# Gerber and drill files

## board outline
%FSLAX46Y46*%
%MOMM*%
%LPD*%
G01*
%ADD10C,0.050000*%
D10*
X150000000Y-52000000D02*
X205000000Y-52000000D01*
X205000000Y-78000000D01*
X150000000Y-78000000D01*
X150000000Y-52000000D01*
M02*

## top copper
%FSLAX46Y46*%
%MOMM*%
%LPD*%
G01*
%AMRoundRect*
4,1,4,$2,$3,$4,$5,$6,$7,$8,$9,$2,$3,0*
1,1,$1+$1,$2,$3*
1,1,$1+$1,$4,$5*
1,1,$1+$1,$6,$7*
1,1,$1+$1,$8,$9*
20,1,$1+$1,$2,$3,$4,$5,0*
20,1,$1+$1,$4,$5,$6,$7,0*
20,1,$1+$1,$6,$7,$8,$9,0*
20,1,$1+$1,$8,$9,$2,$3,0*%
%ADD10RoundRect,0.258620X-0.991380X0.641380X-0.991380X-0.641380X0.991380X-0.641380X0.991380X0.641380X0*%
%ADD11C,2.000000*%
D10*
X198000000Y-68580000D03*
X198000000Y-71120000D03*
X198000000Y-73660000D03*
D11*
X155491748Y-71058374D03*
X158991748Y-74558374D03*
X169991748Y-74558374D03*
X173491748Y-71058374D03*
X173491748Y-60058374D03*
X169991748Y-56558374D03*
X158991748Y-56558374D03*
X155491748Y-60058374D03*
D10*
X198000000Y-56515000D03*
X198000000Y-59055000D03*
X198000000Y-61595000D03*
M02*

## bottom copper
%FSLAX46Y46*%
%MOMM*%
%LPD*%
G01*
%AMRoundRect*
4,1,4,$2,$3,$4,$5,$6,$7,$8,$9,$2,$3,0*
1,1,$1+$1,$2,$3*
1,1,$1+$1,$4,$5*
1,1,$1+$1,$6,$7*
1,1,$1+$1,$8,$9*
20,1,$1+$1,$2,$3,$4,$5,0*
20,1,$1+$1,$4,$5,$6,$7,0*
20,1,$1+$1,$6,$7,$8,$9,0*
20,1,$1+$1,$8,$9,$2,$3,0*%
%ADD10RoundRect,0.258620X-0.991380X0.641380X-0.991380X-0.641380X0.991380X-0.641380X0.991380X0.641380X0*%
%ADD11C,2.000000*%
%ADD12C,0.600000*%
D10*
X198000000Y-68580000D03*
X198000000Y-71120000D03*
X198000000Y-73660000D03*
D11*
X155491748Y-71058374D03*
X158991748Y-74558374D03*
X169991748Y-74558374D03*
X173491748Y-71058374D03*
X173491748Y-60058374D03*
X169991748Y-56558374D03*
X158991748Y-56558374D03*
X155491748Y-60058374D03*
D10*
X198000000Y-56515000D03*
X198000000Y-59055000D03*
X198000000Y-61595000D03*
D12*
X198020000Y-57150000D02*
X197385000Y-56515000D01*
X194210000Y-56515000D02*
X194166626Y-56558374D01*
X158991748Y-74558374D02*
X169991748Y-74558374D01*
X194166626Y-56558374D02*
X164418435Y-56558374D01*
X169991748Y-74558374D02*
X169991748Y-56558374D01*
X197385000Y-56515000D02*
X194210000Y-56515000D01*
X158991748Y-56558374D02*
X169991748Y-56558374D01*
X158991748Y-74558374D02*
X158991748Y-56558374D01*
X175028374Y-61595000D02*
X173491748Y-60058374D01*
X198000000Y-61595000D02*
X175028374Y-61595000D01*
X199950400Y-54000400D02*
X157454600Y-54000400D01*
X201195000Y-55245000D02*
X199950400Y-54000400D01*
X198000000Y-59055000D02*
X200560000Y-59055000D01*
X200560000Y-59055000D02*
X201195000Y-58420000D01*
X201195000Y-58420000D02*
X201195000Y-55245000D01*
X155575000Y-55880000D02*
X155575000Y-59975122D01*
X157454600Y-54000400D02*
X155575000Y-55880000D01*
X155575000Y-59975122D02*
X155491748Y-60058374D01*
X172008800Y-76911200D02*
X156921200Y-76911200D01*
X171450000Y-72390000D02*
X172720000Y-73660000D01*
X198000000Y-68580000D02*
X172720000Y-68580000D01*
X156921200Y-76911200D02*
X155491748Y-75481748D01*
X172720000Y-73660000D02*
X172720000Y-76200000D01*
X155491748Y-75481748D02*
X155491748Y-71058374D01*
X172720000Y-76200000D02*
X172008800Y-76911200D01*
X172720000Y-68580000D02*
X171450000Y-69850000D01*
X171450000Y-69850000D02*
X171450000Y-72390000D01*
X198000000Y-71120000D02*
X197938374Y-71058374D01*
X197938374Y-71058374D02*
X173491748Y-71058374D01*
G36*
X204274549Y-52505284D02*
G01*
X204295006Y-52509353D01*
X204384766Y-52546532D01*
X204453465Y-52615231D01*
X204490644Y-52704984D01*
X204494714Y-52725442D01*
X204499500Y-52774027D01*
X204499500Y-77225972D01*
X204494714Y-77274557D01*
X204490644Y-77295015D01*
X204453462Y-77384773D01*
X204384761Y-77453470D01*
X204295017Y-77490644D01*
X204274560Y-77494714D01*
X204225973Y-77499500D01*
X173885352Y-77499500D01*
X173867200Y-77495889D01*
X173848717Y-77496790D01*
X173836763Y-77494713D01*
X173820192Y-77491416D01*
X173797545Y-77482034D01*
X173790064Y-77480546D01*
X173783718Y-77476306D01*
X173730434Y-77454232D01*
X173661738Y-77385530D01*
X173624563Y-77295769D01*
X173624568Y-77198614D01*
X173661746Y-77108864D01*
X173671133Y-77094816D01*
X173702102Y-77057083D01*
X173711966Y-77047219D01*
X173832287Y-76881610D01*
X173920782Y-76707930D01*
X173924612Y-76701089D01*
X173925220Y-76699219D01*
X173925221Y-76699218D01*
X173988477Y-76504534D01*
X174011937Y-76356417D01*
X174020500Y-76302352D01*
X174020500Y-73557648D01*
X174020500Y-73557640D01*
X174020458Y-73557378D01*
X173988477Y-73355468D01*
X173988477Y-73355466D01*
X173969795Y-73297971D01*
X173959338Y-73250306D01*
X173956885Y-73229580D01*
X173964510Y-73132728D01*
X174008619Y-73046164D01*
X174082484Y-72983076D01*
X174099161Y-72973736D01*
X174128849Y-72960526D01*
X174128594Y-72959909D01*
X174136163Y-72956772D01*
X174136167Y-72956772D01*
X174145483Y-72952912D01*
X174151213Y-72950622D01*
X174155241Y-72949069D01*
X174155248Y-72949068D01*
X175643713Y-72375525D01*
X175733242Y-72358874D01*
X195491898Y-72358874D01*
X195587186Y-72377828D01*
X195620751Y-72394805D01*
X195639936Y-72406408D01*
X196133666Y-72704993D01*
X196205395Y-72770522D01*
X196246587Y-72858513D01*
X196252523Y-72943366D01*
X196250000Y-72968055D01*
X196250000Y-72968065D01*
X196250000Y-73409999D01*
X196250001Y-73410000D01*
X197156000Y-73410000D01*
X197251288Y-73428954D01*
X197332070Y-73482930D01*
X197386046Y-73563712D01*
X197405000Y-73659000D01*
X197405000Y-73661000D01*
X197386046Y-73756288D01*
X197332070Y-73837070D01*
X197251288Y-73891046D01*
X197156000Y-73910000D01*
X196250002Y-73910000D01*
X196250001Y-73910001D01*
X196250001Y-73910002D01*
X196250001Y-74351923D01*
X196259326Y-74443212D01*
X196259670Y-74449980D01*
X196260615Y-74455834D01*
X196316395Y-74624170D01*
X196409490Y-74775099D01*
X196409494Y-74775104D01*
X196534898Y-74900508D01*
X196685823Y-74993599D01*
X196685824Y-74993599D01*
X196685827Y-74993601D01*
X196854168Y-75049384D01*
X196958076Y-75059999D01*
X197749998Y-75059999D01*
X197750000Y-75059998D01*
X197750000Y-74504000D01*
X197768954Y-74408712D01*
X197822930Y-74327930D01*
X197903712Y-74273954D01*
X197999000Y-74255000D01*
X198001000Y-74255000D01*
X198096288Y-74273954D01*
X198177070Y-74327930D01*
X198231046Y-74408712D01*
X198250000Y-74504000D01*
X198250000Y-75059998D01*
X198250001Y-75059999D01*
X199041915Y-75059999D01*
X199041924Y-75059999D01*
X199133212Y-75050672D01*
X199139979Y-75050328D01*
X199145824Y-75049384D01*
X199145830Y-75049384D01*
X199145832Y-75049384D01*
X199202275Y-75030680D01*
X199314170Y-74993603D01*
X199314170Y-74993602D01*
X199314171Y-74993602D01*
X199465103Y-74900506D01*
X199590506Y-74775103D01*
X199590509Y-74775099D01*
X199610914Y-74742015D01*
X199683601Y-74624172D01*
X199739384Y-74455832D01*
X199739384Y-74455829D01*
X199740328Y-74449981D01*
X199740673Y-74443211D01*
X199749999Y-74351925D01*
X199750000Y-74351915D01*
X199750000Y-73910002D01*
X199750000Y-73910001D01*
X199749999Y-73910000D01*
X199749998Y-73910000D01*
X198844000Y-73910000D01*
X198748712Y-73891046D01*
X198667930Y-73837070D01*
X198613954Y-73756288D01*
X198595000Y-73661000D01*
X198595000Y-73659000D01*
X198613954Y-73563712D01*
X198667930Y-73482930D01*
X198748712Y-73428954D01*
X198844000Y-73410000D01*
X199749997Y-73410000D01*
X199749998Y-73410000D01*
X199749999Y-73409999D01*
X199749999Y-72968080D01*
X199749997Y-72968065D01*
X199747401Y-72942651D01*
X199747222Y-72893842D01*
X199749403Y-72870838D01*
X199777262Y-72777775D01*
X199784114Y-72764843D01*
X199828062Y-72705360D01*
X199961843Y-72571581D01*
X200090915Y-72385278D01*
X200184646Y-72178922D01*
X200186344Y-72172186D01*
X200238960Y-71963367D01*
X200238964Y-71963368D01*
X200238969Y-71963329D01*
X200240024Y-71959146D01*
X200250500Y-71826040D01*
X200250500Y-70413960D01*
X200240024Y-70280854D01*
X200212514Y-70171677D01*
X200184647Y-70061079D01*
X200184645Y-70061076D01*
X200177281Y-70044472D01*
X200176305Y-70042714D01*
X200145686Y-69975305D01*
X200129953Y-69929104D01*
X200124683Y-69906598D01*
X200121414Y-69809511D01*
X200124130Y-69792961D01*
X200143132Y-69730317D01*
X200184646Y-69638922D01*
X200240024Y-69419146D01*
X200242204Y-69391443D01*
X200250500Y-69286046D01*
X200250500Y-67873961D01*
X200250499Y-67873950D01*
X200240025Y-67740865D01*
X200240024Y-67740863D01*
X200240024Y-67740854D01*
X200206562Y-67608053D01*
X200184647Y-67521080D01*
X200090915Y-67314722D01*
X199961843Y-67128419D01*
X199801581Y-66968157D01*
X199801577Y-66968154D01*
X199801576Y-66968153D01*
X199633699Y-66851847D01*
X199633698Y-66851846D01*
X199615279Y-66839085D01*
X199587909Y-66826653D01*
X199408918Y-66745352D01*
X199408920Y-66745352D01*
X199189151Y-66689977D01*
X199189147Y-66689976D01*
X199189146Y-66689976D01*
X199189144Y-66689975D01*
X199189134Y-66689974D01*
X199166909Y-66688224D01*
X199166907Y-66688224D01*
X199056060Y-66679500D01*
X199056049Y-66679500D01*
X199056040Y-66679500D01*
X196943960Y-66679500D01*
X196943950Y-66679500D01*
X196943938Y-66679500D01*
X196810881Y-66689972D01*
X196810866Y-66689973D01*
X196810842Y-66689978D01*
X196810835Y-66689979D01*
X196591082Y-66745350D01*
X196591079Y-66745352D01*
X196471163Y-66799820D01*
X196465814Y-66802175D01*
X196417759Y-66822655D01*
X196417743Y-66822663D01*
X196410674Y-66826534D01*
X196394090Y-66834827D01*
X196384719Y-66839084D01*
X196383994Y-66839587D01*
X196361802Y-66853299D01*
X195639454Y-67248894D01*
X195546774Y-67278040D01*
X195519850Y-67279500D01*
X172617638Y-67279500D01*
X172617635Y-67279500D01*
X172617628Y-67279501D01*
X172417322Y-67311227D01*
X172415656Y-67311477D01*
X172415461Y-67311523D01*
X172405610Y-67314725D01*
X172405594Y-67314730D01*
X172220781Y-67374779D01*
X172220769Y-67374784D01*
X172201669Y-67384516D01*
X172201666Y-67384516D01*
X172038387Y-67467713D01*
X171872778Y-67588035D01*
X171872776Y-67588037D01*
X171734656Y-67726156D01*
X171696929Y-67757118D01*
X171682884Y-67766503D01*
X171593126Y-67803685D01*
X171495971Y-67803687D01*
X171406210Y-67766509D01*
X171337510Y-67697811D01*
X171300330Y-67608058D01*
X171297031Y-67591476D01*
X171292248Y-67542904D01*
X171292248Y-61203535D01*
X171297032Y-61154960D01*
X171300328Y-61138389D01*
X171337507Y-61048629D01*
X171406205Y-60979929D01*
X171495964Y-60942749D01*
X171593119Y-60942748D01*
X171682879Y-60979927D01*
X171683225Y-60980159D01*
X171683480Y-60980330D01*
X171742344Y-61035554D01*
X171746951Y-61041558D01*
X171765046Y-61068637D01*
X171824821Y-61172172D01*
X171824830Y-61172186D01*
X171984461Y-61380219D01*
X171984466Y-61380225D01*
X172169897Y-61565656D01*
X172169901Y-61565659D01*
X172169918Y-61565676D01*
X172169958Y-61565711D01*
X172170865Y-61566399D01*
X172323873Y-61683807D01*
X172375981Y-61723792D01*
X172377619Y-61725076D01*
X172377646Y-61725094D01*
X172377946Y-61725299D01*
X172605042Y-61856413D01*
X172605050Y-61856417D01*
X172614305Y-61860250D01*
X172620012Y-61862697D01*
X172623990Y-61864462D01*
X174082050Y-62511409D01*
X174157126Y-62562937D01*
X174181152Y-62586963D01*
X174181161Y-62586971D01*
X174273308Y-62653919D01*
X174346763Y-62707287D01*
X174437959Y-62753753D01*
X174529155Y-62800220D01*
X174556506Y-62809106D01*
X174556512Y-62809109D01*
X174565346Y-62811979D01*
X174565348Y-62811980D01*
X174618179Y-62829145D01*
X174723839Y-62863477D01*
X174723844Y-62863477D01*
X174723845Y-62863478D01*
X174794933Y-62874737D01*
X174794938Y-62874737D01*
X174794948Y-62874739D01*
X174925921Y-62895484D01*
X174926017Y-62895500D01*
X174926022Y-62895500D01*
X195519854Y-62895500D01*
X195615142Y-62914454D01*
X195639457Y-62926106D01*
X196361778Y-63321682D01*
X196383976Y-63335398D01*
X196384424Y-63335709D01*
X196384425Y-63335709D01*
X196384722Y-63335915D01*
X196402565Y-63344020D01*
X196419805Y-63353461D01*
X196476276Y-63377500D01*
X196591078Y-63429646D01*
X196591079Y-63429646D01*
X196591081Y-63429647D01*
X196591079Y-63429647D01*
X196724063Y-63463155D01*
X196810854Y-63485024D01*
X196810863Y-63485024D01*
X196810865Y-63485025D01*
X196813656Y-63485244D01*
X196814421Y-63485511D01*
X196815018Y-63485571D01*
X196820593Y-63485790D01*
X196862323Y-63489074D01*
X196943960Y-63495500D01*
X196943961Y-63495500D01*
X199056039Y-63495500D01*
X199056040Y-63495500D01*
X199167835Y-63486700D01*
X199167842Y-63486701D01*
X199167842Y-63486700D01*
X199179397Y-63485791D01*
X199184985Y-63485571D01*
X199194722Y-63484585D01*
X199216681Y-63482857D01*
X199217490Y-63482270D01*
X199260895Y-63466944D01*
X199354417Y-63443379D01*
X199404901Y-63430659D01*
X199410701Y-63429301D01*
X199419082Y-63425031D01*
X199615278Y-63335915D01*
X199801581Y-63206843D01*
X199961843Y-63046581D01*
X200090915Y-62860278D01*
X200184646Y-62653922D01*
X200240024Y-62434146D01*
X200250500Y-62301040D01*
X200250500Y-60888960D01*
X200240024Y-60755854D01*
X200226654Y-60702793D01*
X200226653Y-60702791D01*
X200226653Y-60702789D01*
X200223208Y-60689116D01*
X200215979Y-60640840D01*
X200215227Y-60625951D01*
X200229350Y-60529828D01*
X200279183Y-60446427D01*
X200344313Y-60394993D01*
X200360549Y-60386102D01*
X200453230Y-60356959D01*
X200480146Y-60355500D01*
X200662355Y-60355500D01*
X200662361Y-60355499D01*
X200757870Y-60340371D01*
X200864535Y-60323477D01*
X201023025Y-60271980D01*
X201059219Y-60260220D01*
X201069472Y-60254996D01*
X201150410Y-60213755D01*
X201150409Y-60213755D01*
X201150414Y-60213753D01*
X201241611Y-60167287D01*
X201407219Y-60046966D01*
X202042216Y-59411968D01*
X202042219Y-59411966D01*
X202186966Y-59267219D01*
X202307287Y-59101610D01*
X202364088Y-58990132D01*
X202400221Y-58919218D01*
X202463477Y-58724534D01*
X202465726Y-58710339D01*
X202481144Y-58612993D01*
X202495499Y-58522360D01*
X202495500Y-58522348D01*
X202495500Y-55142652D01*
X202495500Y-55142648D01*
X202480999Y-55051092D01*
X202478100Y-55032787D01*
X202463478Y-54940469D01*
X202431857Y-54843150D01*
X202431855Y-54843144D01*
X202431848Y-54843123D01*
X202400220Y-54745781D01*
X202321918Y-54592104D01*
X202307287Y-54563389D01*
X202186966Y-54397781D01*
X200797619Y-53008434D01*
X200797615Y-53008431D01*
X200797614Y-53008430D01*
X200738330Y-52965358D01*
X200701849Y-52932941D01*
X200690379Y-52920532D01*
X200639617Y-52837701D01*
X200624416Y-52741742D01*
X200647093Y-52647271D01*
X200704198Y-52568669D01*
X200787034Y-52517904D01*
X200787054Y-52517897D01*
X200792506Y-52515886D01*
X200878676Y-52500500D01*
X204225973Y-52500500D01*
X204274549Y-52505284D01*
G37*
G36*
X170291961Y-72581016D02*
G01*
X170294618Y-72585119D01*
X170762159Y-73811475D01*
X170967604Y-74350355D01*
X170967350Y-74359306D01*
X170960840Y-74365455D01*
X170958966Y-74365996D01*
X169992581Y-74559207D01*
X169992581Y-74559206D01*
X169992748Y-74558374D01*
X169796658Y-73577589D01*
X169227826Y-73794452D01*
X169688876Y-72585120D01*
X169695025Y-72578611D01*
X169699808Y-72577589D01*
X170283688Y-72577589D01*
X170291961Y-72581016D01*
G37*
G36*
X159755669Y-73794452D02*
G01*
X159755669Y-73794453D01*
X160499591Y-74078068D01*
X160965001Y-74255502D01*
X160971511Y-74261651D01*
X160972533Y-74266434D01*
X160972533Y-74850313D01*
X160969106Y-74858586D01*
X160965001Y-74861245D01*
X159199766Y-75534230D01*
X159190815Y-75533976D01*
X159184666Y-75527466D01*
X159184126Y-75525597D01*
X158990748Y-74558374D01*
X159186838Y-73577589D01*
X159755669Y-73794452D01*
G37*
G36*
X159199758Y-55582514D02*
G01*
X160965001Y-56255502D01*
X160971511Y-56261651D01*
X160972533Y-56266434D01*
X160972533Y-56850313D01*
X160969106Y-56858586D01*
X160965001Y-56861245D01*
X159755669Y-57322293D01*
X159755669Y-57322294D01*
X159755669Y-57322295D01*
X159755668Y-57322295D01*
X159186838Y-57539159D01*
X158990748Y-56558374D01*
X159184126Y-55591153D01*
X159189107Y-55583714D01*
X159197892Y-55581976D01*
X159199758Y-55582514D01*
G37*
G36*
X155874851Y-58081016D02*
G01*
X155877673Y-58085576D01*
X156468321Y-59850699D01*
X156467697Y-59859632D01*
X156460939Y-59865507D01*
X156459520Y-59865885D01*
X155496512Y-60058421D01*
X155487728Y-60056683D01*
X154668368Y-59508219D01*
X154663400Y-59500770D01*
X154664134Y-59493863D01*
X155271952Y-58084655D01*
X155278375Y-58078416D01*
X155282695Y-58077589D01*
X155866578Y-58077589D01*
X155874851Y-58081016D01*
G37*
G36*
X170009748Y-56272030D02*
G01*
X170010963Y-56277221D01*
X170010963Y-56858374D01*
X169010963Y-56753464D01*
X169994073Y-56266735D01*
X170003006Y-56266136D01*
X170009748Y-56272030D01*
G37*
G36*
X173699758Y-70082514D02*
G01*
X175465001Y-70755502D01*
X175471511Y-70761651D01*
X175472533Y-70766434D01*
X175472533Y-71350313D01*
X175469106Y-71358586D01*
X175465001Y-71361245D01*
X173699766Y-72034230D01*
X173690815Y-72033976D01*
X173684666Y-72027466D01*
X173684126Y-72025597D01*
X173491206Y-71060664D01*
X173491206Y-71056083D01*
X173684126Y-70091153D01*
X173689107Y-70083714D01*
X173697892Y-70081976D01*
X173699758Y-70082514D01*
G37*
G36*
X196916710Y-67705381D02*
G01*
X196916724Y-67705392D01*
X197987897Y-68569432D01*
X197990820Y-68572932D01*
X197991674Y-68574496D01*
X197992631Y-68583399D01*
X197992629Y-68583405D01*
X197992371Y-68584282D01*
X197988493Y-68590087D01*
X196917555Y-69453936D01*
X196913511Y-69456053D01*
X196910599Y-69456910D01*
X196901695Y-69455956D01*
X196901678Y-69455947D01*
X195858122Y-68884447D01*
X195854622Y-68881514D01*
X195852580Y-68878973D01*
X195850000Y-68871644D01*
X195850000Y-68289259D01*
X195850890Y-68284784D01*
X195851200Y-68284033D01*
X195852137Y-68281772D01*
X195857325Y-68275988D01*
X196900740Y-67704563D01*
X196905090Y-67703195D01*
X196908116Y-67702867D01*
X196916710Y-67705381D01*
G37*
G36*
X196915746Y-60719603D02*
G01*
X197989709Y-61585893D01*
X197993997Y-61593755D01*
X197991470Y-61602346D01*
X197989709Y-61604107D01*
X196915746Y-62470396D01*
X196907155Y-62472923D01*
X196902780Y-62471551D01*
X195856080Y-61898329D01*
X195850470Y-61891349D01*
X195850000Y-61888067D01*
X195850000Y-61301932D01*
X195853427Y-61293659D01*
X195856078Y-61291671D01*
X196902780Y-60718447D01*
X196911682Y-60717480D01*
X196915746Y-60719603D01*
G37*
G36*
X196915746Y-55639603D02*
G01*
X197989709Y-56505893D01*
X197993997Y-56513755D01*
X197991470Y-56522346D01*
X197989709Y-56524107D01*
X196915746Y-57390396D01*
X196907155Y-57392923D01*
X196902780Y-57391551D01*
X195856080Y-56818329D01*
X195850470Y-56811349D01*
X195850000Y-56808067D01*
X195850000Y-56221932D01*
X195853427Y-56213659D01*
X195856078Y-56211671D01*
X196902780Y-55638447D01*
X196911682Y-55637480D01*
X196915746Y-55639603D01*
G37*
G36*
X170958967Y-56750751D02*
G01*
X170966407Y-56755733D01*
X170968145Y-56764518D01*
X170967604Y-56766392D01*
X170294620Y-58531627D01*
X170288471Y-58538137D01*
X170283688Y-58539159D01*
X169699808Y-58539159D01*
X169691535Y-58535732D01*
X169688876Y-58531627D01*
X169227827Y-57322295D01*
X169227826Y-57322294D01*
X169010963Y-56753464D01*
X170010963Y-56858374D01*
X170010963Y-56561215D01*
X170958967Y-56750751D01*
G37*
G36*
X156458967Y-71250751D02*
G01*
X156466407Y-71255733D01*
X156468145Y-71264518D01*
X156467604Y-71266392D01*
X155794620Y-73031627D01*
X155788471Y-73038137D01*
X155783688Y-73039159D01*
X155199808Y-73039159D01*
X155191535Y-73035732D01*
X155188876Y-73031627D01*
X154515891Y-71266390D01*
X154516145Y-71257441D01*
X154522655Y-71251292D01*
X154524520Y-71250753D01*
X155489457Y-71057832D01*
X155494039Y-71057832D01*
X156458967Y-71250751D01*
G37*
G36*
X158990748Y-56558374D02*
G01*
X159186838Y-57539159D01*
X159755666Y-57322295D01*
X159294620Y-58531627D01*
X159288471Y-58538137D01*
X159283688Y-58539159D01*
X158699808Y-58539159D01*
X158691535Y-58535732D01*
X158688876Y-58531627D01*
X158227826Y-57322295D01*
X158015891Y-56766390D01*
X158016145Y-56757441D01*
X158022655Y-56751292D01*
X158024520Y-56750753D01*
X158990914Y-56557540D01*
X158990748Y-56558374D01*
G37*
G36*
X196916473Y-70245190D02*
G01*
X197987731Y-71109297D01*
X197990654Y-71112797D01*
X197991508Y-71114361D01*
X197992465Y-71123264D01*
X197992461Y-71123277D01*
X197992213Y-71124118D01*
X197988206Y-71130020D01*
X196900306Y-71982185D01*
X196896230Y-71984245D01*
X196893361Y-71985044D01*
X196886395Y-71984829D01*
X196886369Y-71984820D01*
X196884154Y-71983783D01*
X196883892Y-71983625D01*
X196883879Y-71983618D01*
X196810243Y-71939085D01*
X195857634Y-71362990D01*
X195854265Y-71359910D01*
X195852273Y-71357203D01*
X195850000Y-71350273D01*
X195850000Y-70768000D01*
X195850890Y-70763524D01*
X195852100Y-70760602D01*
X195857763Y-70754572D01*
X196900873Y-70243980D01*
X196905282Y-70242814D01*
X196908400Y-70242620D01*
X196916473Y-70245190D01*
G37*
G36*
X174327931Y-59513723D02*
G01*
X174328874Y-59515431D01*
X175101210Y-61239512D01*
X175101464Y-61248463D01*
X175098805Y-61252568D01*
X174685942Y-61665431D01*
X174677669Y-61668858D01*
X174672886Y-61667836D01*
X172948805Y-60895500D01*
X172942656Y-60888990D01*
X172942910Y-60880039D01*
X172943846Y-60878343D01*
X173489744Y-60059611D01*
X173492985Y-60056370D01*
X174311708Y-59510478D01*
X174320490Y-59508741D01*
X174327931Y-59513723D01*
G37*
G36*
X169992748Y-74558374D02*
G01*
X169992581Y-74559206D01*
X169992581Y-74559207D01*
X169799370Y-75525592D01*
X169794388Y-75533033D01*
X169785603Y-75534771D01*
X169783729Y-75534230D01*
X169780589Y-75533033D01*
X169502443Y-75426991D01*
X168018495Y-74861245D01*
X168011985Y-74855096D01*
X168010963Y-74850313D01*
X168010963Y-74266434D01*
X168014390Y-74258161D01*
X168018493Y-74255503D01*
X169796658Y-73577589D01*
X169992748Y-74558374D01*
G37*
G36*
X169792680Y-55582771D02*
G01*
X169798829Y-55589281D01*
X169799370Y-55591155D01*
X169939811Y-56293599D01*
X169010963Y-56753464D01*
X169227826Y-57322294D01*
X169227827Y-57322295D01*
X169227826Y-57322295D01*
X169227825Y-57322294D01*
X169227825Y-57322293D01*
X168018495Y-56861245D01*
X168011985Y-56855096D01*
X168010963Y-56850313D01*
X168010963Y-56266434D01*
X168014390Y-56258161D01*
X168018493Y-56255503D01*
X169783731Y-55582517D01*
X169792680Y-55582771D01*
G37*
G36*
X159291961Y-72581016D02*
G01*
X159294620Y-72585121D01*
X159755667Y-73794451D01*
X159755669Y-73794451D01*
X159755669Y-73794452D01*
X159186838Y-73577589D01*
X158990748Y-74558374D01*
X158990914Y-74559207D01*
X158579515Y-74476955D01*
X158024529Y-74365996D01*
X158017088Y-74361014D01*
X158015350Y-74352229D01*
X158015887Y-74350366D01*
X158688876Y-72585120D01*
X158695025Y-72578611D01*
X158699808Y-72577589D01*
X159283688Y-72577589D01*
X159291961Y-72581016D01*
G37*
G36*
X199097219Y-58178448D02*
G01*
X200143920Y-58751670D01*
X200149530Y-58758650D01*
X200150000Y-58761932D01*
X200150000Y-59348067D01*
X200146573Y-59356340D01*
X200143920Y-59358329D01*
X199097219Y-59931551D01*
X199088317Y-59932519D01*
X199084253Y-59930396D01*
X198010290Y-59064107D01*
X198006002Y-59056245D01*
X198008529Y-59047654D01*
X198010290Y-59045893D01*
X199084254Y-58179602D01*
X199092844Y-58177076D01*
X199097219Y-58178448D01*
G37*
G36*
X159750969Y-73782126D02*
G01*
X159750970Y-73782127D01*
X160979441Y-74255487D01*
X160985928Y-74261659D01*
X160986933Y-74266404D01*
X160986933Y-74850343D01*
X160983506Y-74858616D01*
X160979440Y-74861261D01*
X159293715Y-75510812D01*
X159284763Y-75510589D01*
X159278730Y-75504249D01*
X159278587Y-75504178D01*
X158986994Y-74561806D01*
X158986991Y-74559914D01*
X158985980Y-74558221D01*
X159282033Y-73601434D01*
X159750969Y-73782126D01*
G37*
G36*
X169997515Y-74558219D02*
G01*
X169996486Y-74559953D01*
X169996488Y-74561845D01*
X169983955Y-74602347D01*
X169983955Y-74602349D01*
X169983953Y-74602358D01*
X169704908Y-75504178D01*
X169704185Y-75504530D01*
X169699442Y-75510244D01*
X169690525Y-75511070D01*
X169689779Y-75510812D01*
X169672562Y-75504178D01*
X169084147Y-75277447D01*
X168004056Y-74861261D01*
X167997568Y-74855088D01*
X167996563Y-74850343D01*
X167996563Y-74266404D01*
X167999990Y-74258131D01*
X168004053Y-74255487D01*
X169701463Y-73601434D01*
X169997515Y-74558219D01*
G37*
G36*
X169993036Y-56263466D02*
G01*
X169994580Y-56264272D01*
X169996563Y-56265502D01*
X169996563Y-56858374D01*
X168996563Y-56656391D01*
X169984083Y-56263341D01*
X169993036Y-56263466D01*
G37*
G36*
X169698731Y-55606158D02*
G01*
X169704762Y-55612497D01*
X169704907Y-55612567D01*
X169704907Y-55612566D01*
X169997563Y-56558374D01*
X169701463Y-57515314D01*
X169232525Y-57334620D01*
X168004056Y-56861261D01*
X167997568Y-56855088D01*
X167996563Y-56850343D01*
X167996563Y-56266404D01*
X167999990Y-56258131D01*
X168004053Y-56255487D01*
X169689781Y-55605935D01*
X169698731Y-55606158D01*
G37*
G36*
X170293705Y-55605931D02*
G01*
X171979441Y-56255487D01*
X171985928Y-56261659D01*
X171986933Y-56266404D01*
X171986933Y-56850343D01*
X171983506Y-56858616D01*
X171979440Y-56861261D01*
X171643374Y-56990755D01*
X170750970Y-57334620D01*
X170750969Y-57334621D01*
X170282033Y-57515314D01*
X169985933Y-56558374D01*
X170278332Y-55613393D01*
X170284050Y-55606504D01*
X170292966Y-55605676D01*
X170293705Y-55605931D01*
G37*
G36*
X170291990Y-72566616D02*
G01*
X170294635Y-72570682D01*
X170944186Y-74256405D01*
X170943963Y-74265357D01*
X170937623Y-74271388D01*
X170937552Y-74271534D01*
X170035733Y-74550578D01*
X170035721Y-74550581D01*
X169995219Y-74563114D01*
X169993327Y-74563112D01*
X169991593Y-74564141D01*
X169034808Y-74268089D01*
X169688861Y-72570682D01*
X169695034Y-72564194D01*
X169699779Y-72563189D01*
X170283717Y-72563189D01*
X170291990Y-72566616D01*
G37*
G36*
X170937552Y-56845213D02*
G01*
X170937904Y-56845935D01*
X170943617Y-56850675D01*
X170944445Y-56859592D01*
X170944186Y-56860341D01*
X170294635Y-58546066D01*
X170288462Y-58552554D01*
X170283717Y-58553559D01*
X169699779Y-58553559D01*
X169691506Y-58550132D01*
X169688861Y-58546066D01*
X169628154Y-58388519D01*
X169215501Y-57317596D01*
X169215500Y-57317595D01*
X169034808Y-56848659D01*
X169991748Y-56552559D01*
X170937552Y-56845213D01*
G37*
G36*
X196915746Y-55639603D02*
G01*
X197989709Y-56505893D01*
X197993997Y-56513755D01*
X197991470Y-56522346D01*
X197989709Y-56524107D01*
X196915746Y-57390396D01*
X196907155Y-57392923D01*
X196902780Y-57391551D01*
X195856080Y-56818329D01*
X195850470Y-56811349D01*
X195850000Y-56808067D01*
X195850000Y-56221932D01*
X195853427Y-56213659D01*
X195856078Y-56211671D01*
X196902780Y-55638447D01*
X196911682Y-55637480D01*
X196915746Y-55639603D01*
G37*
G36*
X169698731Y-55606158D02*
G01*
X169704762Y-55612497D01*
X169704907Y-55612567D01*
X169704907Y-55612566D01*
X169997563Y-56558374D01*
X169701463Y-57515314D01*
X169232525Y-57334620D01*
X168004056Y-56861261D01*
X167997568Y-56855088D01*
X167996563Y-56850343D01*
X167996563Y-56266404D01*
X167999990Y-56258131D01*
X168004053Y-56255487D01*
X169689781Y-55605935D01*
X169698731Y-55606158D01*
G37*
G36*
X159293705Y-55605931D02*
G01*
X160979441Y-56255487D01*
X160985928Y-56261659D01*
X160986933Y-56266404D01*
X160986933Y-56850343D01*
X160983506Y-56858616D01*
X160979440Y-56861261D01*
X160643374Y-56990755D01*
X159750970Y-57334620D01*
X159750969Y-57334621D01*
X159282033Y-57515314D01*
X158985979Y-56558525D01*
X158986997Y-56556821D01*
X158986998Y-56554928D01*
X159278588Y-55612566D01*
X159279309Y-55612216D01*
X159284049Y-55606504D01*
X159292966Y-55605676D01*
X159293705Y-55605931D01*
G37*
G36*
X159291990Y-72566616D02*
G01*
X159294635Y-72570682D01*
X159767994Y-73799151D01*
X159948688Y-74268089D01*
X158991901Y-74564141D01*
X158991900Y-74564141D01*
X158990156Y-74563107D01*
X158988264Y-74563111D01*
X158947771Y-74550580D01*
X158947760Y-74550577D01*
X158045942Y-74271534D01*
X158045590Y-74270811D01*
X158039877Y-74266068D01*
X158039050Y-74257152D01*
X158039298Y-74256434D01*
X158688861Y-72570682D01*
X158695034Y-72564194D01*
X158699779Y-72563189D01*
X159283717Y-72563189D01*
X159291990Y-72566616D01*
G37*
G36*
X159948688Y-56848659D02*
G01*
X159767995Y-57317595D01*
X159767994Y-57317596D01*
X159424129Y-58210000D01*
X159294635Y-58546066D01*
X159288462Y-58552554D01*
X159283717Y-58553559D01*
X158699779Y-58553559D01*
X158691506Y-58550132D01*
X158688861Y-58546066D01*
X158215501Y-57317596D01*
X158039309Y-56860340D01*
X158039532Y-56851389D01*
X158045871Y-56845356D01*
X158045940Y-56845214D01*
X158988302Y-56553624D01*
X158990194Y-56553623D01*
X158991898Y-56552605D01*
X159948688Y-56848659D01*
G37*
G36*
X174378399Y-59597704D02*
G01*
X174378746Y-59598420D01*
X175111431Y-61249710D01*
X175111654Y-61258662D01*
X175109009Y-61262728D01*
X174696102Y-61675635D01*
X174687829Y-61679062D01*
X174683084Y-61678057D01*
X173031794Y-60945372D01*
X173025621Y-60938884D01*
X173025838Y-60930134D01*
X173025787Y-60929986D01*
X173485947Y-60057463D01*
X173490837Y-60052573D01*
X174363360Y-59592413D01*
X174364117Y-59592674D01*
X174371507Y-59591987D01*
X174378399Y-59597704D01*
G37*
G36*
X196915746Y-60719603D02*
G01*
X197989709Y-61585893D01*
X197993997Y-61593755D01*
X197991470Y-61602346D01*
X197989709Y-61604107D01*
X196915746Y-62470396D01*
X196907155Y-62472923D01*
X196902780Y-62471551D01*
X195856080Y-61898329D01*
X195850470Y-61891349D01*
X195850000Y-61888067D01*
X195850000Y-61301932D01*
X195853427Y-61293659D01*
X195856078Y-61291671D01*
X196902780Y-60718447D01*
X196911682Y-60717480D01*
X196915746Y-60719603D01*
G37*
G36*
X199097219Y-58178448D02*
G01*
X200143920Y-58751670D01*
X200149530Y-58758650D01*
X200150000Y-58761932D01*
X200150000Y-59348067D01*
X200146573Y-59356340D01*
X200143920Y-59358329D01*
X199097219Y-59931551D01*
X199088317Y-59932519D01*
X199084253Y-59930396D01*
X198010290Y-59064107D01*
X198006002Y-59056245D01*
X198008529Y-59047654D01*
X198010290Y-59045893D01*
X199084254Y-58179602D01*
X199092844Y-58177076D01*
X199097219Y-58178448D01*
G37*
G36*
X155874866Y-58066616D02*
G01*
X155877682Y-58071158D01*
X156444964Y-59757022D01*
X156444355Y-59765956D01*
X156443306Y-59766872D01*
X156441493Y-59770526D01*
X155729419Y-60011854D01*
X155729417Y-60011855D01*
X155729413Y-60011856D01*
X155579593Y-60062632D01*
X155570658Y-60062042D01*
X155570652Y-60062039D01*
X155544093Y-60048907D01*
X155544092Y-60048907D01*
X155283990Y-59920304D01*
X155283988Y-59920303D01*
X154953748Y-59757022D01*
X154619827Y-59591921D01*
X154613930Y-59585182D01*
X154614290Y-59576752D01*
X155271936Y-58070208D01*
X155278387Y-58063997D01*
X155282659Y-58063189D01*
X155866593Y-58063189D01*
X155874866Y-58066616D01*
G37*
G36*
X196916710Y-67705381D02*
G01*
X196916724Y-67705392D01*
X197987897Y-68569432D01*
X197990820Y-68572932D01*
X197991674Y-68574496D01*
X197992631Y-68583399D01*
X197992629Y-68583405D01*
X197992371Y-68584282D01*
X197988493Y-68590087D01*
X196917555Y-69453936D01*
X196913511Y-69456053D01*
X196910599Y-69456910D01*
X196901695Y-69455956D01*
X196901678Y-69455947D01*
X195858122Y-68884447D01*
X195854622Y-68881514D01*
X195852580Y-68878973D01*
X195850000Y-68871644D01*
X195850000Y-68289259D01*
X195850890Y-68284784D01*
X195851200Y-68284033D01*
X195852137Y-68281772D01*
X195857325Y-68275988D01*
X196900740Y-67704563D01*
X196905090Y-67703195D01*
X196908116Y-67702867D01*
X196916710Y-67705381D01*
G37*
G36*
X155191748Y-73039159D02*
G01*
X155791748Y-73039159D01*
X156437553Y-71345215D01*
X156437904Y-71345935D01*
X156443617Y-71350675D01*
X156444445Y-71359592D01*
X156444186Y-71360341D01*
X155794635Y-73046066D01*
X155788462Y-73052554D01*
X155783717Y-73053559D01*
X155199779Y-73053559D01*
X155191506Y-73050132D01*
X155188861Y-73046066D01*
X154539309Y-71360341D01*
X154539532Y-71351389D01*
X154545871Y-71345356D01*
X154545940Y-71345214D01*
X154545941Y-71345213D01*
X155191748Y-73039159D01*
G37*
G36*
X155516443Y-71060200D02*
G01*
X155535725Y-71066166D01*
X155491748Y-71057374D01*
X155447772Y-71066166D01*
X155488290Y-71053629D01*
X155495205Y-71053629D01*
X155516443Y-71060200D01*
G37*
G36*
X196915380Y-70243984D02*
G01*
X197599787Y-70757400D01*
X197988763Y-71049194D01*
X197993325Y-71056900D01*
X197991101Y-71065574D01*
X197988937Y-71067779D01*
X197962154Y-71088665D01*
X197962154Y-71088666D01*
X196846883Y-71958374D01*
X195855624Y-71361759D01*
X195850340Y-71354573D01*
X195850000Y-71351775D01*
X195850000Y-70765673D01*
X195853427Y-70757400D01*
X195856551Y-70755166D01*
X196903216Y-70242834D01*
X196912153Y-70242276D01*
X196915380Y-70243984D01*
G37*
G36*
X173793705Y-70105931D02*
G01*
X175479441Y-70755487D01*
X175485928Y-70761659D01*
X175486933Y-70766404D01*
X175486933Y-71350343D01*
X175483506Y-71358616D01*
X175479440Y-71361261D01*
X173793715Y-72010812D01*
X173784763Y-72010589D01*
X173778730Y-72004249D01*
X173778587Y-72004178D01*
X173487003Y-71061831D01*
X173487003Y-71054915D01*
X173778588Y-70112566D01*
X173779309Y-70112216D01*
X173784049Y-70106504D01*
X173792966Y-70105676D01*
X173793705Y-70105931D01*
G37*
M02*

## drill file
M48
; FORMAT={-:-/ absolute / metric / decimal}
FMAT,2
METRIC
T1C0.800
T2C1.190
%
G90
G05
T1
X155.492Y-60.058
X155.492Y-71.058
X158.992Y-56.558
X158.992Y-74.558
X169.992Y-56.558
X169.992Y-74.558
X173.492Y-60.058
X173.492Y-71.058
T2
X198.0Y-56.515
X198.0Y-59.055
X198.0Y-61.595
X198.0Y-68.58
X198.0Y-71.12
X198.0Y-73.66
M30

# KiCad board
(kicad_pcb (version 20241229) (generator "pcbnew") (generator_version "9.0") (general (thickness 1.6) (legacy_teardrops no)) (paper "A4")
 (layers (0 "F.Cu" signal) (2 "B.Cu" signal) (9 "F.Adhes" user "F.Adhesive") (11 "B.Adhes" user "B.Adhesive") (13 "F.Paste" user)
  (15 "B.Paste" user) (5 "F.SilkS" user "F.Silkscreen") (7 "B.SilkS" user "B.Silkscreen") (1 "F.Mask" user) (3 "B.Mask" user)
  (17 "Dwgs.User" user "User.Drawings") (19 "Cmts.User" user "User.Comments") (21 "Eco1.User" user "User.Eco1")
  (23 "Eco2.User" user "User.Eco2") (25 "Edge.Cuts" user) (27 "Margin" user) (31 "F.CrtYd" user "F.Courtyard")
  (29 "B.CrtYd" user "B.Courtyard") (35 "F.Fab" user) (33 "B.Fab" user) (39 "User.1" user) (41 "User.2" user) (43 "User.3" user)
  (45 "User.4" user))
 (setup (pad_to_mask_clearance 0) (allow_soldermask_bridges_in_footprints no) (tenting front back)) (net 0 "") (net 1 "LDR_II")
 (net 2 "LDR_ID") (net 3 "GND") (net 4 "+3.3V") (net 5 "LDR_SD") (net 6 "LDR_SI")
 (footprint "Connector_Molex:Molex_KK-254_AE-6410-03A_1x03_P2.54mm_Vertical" (layer "F.Cu") (at 198 68.58 -90)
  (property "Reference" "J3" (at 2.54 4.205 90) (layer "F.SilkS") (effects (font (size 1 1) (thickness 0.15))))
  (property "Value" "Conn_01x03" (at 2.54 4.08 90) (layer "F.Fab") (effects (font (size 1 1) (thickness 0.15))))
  (pad "1" thru_hole roundrect (at 0 0 270) (size 1.8 2.5) (drill 1.19) (layers "*.Cu" "*.Mask") (remove_unused_layers no)
   (roundrect_rratio 0.143678) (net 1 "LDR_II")
   (teardrops (best_length_ratio 0.5) (max_length 1) (best_width_ratio 1) (max_width 2) (curved_edges no) (filter_ratio 0.9) (enabled yes)
    (allow_two_segments yes) (prefer_zone_connections yes)))
  (pad "2" thru_hole roundrect (at 2.54 0 270) (size 1.8 2.5) (drill 1.19) (layers "*.Cu" "*.Mask") (remove_unused_layers no)
   (roundrect_rratio 0.143678) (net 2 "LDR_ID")
   (teardrops (best_length_ratio 0.5) (max_length 1) (best_width_ratio 1) (max_width 2) (curved_edges no) (filter_ratio 0.9) (enabled yes)
    (allow_two_segments yes) (prefer_zone_connections yes)))
  (pad "3" thru_hole roundrect (at 5.08 0 270) (size 1.8 2.5) (drill 1.19) (layers "*.Cu" "*.Mask") (remove_unused_layers no)
   (roundrect_rratio 0.143678) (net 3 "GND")
   (teardrops (best_length_ratio 0.5) (max_length 1) (best_width_ratio 1) (max_width 2) (curved_edges no) (filter_ratio 0.9) (enabled yes)
    (allow_two_segments yes) (prefer_zone_connections yes))))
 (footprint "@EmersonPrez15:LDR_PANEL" (layer "F.Cu") (at 164.991748 65.558374)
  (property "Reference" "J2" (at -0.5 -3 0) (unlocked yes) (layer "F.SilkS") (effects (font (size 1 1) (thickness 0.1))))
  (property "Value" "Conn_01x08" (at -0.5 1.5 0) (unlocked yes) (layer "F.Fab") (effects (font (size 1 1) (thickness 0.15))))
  (pad "1" thru_hole circle (at -9.5 5.5 180) (size 2 2) (drill 0.8) (layers "*.Cu" "*.Mask") (remove_unused_layers no) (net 1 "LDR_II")
   (teardrops (best_length_ratio 0.5) (max_length 1) (best_width_ratio 1) (max_width 2) (curved_edges no) (filter_ratio 0.9) (enabled yes)
    (allow_two_segments yes) (prefer_zone_connections yes)))
  (pad "2" thru_hole circle (at -6 9 90) (size 2 2) (drill 0.8) (layers "*.Cu" "*.Mask") (remove_unused_layers no) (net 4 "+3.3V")
   (teardrops (best_length_ratio 0.5) (max_length 1) (best_width_ratio 1) (max_width 2) (curved_edges no) (filter_ratio 0.9) (enabled yes)
    (allow_two_segments yes) (prefer_zone_connections yes)))
  (pad "3" thru_hole circle (at 5 9 90) (size 2 2) (drill 0.8) (layers "*.Cu" "*.Mask") (remove_unused_layers no) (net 4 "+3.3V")
   (teardrops (best_length_ratio 0.5) (max_length 1) (best_width_ratio 1) (max_width 2) (curved_edges no) (filter_ratio 0.9) (enabled yes)
    (allow_two_segments yes) (prefer_zone_connections yes)))
  (pad "4" thru_hole circle (at 8.5 5.5 180) (size 2 2) (drill 0.8) (layers "*.Cu" "*.Mask") (remove_unused_layers no) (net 2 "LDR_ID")
   (teardrops (best_length_ratio 0.5) (max_length 1) (best_width_ratio 1) (max_width 2) (curved_edges no) (filter_ratio 0.9) (enabled yes)
    (allow_two_segments yes) (prefer_zone_connections yes)))
  (pad "5" thru_hole circle (at 8.5 -5.5 180) (size 2 2) (drill 0.8) (layers "*.Cu" "*.Mask") (remove_unused_layers no) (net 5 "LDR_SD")
   (teardrops (best_length_ratio 0.5) (max_length 1) (best_width_ratio 1) (max_width 2) (curved_edges no) (filter_ratio 0.9) (enabled yes)
    (allow_two_segments yes) (prefer_zone_connections yes)))
  (pad "6" thru_hole circle (at 5 -9 90) (size 2 2) (drill 0.8) (layers "*.Cu" "*.Mask") (remove_unused_layers no) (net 4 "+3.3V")
   (teardrops (best_length_ratio 0.5) (max_length 1) (best_width_ratio 1) (max_width 2) (curved_edges no) (filter_ratio 0.9) (enabled yes)
    (allow_two_segments yes) (prefer_zone_connections yes)))
  (pad "7" thru_hole circle (at -6 -9 90) (size 2 2) (drill 0.8) (layers "*.Cu" "*.Mask") (remove_unused_layers no) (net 4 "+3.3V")
   (teardrops (best_length_ratio 0.5) (max_length 1) (best_width_ratio 1) (max_width 2) (curved_edges no) (filter_ratio 0.9) (enabled yes)
    (allow_two_segments yes) (prefer_zone_connections yes)))
  (pad "8" thru_hole circle (at -9.5 -5.5 180) (size 2 2) (drill 0.8) (layers "*.Cu" "*.Mask") (remove_unused_layers no) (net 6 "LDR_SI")
   (teardrops (best_length_ratio 0.5) (max_length 1) (best_width_ratio 1) (max_width 2) (curved_edges no) (filter_ratio 0.9) (enabled yes)
    (allow_two_segments yes) (prefer_zone_connections yes))))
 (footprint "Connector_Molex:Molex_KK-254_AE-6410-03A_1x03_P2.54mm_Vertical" (layer "F.Cu") (at 198 56.515 -90)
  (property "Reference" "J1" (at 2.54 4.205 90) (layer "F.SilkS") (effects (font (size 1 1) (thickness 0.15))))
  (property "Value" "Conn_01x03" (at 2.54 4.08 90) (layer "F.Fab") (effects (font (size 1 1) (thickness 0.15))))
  (pad "1" thru_hole roundrect (at 0 0 270) (size 1.8 2.5) (drill 1.19) (layers "*.Cu" "*.Mask") (remove_unused_layers no)
   (roundrect_rratio 0.143678) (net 4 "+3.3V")
   (teardrops (best_length_ratio 0.5) (max_length 1) (best_width_ratio 1) (max_width 2) (curved_edges no) (filter_ratio 0.9) (enabled yes)
    (allow_two_segments yes) (prefer_zone_connections yes)))
  (pad "2" thru_hole roundrect (at 2.54 0 270) (size 1.8 2.5) (drill 1.19) (layers "*.Cu" "*.Mask") (remove_unused_layers no)
   (roundrect_rratio 0.143678) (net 6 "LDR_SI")
   (teardrops (best_length_ratio 0.5) (max_length 1) (best_width_ratio 1) (max_width 2) (curved_edges no) (filter_ratio 0.9) (enabled yes)
    (allow_two_segments yes) (prefer_zone_connections yes)))
  (pad "3" thru_hole roundrect (at 5.08 0 270) (size 1.8 2.5) (drill 1.19) (layers "*.Cu" "*.Mask") (remove_unused_layers no)
   (roundrect_rratio 0.143678) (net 5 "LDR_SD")
   (teardrops (best_length_ratio 0.5) (max_length 1) (best_width_ratio 1) (max_width 2) (curved_edges no) (filter_ratio 0.9) (enabled yes)
    (allow_two_segments yes) (prefer_zone_connections yes))))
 (gr_rect (start 150 52) (end 205 78) (stroke (width 0.05) (type default)) (fill no) (layer "Edge.Cuts"))
 (segment (start 198.02 57.15) (end 197.385 56.515) (width 0.6) (layer "B.Cu") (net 4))
 (segment (start 194.21 56.515) (end 194.166626 56.558374) (width 0.6) (layer "B.Cu") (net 4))
 (segment (start 158.991748 74.558374) (end 169.991748 74.558374) (width 0.6) (layer "B.Cu") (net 4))
 (segment (start 194.166626 56.558374) (end 164.418435 56.558374) (width 0.6) (layer "B.Cu") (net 4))
 (segment (start 169.991748 74.558374) (end 169.991748 56.558374) (width 0.6) (layer "B.Cu") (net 4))
 (segment (start 197.385 56.515) (end 194.21 56.515) (width 0.6) (layer "B.Cu") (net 4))
 (segment (start 158.991748 56.558374) (end 169.991748 56.558374) (width 0.6) (layer "B.Cu") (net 4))
 (segment (start 158.991748 74.558374) (end 158.991748 56.558374) (width 0.6) (layer "B.Cu") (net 4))
 (segment (start 175.028374 61.595) (end 173.491748 60.058374) (width 0.6) (layer "B.Cu") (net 5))
 (segment (start 198 61.595) (end 175.028374 61.595) (width 0.6) (layer "B.Cu") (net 5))
 (segment (start 199.9504 54.0004) (end 157.4546 54.0004) (width 0.6) (layer "B.Cu") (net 6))
 (segment (start 201.195 55.245) (end 199.9504 54.0004) (width 0.6) (layer "B.Cu") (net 6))
 (segment (start 198 59.055) (end 200.56 59.055) (width 0.6) (layer "B.Cu") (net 6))
 (segment (start 200.56 59.055) (end 201.195 58.42) (width 0.6) (layer "B.Cu") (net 6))
 (segment (start 201.195 58.42) (end 201.195 55.245) (width 0.6) (layer "B.Cu") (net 6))
 (segment (start 155.575 55.88) (end 155.575 59.975122) (width 0.6) (layer "B.Cu") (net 6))
 (segment (start 157.4546 54.0004) (end 155.575 55.88) (width 0.6) (layer "B.Cu") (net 6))
 (segment (start 155.575 59.975122) (end 155.491748 60.058374) (width 0.6) (layer "B.Cu") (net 6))
 (segment (start 172.0088 76.9112) (end 156.9212 76.9112) (width 0.6) (layer "B.Cu") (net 1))
 (segment (start 171.45 72.39) (end 172.72 73.66) (width 0.6) (layer "B.Cu") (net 1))
 (segment (start 198 68.58) (end 172.72 68.58) (width 0.6) (layer "B.Cu") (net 1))
 (segment (start 156.9212 76.9112) (end 155.491748 75.481748) (width 0.6) (layer "B.Cu") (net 1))
 (segment (start 172.72 73.66) (end 172.72 76.2) (width 0.6) (layer "B.Cu") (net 1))
 (segment (start 155.491748 75.481748) (end 155.491748 71.058374) (width 0.6) (layer "B.Cu") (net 1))
 (segment (start 172.72 76.2) (end 172.0088 76.9112) (width 0.6) (layer "B.Cu") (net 1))
 (segment (start 172.72 68.58) (end 171.45 69.85) (width 0.6) (layer "B.Cu") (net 1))
 (segment (start 171.45 69.85) (end 171.45 72.39) (width 0.6) (layer "B.Cu") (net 1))
 (segment (start 198 71.12) (end 197.938374 71.058374) (width 0.6) (layer "B.Cu") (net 2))
 (segment (start 197.938374 71.058374) (end 173.491748 71.058374) (width 0.6) (layer "B.Cu") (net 2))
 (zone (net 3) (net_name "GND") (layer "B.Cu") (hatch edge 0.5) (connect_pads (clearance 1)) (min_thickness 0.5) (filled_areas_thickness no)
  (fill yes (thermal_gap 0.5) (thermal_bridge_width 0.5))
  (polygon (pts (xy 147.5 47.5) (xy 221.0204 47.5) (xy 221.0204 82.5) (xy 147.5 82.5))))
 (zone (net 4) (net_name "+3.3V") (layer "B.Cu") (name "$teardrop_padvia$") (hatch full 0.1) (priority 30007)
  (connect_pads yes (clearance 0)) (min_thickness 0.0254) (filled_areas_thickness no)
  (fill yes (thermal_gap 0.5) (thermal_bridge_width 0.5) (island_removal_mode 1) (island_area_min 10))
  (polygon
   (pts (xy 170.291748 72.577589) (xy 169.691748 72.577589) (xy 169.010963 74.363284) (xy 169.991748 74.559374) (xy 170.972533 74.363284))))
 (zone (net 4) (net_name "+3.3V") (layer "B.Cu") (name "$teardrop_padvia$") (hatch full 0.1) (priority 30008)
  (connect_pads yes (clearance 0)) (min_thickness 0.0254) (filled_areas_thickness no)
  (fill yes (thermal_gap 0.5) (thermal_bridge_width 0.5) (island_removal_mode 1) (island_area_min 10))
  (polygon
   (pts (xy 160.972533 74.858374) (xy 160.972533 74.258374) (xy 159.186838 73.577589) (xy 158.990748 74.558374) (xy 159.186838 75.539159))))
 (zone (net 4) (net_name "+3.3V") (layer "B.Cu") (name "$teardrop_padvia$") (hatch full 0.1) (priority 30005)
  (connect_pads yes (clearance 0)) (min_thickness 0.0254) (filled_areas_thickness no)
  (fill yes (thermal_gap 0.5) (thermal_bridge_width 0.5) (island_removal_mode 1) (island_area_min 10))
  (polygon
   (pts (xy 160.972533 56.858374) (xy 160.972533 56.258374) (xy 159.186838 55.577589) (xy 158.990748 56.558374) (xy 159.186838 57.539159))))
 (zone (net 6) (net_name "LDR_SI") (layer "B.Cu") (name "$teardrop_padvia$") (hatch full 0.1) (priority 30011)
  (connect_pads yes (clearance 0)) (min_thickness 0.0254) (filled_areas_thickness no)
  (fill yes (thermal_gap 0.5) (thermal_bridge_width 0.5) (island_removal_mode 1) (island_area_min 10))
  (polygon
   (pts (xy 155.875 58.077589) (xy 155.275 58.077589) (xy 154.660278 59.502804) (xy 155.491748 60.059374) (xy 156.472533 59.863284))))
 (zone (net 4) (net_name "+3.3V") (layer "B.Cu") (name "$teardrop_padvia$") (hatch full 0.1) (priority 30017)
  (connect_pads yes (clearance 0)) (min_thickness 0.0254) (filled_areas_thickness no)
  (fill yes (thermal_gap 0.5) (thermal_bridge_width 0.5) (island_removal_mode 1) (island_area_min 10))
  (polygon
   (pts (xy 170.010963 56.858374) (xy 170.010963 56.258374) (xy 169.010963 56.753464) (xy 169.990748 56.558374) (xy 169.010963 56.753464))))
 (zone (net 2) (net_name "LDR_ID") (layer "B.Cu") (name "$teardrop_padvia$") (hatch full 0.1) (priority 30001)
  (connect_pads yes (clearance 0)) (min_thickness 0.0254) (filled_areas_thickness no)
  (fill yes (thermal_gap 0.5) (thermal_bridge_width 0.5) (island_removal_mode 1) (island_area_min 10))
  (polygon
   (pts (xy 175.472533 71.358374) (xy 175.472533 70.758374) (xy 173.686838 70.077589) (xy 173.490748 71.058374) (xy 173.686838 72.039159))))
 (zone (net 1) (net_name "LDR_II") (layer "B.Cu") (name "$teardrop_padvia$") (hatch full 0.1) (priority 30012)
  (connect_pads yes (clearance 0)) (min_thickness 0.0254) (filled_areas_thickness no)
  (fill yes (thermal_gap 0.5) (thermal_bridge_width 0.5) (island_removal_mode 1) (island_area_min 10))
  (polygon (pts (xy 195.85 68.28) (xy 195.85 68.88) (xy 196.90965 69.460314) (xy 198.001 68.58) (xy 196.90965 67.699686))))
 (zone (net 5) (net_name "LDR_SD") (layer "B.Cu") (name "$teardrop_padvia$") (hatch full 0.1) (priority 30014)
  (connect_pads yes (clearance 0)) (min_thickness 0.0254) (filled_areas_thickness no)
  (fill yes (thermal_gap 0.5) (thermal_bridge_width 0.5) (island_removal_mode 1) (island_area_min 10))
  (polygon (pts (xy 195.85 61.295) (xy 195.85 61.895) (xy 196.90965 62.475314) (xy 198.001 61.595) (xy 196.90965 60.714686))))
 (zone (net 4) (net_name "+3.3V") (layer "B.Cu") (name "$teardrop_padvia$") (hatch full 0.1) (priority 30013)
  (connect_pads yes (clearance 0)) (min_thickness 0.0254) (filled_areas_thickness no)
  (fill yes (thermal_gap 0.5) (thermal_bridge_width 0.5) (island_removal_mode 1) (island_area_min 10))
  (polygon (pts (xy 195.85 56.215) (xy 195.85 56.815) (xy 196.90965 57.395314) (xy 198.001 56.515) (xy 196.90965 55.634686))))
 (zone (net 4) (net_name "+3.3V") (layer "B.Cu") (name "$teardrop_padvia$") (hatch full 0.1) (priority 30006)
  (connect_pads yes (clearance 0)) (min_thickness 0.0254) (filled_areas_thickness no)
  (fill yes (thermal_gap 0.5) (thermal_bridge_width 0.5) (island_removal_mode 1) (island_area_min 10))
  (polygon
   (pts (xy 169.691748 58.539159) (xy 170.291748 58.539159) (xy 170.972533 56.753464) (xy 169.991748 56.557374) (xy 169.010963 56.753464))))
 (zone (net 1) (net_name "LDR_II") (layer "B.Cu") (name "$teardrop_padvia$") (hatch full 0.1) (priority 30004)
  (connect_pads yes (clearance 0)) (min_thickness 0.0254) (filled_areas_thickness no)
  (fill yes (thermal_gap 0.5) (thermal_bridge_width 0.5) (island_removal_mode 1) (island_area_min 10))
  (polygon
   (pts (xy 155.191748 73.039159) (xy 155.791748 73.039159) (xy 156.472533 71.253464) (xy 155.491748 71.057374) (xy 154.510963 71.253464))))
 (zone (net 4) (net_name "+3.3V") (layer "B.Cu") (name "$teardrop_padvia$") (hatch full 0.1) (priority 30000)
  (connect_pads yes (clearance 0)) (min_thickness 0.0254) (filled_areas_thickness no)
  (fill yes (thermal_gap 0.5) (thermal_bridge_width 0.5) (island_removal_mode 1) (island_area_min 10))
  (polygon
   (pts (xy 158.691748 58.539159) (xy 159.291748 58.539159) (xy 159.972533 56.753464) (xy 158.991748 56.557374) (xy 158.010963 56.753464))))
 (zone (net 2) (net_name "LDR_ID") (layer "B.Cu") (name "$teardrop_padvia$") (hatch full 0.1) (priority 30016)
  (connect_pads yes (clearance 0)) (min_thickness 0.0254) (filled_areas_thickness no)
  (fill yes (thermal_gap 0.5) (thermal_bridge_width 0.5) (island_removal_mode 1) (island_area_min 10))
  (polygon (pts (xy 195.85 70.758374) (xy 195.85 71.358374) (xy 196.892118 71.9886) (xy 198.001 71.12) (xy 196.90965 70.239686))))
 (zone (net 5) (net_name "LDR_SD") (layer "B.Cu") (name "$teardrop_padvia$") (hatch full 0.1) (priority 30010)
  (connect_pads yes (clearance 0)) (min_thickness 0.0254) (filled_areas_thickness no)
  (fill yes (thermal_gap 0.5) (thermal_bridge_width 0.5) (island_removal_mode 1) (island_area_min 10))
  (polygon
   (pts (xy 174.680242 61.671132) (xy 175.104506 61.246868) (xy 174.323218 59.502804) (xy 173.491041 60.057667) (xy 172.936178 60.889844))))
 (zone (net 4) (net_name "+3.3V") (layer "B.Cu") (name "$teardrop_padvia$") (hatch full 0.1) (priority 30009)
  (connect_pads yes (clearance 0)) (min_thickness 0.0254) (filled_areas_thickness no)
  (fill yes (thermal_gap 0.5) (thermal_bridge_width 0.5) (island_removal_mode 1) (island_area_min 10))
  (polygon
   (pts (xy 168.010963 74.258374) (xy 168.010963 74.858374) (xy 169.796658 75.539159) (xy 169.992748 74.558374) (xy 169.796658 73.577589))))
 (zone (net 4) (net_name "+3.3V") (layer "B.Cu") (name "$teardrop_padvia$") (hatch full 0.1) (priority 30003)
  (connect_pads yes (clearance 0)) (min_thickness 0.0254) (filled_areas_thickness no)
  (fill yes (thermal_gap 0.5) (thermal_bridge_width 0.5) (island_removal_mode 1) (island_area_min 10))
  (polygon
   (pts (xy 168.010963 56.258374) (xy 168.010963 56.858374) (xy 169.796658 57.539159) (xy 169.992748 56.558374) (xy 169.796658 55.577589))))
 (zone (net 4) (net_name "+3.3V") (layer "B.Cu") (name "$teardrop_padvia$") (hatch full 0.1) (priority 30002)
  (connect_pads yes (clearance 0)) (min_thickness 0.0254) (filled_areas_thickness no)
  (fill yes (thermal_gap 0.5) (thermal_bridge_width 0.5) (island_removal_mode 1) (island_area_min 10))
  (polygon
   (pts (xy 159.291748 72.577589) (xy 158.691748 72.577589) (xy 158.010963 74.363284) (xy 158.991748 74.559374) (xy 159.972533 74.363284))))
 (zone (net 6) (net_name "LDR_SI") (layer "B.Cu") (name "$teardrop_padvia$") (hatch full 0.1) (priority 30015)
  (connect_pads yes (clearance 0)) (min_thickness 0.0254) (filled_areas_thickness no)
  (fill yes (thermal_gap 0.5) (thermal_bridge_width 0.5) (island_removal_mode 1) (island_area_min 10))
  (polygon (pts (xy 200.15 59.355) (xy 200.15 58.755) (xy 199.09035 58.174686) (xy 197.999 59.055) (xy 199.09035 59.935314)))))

